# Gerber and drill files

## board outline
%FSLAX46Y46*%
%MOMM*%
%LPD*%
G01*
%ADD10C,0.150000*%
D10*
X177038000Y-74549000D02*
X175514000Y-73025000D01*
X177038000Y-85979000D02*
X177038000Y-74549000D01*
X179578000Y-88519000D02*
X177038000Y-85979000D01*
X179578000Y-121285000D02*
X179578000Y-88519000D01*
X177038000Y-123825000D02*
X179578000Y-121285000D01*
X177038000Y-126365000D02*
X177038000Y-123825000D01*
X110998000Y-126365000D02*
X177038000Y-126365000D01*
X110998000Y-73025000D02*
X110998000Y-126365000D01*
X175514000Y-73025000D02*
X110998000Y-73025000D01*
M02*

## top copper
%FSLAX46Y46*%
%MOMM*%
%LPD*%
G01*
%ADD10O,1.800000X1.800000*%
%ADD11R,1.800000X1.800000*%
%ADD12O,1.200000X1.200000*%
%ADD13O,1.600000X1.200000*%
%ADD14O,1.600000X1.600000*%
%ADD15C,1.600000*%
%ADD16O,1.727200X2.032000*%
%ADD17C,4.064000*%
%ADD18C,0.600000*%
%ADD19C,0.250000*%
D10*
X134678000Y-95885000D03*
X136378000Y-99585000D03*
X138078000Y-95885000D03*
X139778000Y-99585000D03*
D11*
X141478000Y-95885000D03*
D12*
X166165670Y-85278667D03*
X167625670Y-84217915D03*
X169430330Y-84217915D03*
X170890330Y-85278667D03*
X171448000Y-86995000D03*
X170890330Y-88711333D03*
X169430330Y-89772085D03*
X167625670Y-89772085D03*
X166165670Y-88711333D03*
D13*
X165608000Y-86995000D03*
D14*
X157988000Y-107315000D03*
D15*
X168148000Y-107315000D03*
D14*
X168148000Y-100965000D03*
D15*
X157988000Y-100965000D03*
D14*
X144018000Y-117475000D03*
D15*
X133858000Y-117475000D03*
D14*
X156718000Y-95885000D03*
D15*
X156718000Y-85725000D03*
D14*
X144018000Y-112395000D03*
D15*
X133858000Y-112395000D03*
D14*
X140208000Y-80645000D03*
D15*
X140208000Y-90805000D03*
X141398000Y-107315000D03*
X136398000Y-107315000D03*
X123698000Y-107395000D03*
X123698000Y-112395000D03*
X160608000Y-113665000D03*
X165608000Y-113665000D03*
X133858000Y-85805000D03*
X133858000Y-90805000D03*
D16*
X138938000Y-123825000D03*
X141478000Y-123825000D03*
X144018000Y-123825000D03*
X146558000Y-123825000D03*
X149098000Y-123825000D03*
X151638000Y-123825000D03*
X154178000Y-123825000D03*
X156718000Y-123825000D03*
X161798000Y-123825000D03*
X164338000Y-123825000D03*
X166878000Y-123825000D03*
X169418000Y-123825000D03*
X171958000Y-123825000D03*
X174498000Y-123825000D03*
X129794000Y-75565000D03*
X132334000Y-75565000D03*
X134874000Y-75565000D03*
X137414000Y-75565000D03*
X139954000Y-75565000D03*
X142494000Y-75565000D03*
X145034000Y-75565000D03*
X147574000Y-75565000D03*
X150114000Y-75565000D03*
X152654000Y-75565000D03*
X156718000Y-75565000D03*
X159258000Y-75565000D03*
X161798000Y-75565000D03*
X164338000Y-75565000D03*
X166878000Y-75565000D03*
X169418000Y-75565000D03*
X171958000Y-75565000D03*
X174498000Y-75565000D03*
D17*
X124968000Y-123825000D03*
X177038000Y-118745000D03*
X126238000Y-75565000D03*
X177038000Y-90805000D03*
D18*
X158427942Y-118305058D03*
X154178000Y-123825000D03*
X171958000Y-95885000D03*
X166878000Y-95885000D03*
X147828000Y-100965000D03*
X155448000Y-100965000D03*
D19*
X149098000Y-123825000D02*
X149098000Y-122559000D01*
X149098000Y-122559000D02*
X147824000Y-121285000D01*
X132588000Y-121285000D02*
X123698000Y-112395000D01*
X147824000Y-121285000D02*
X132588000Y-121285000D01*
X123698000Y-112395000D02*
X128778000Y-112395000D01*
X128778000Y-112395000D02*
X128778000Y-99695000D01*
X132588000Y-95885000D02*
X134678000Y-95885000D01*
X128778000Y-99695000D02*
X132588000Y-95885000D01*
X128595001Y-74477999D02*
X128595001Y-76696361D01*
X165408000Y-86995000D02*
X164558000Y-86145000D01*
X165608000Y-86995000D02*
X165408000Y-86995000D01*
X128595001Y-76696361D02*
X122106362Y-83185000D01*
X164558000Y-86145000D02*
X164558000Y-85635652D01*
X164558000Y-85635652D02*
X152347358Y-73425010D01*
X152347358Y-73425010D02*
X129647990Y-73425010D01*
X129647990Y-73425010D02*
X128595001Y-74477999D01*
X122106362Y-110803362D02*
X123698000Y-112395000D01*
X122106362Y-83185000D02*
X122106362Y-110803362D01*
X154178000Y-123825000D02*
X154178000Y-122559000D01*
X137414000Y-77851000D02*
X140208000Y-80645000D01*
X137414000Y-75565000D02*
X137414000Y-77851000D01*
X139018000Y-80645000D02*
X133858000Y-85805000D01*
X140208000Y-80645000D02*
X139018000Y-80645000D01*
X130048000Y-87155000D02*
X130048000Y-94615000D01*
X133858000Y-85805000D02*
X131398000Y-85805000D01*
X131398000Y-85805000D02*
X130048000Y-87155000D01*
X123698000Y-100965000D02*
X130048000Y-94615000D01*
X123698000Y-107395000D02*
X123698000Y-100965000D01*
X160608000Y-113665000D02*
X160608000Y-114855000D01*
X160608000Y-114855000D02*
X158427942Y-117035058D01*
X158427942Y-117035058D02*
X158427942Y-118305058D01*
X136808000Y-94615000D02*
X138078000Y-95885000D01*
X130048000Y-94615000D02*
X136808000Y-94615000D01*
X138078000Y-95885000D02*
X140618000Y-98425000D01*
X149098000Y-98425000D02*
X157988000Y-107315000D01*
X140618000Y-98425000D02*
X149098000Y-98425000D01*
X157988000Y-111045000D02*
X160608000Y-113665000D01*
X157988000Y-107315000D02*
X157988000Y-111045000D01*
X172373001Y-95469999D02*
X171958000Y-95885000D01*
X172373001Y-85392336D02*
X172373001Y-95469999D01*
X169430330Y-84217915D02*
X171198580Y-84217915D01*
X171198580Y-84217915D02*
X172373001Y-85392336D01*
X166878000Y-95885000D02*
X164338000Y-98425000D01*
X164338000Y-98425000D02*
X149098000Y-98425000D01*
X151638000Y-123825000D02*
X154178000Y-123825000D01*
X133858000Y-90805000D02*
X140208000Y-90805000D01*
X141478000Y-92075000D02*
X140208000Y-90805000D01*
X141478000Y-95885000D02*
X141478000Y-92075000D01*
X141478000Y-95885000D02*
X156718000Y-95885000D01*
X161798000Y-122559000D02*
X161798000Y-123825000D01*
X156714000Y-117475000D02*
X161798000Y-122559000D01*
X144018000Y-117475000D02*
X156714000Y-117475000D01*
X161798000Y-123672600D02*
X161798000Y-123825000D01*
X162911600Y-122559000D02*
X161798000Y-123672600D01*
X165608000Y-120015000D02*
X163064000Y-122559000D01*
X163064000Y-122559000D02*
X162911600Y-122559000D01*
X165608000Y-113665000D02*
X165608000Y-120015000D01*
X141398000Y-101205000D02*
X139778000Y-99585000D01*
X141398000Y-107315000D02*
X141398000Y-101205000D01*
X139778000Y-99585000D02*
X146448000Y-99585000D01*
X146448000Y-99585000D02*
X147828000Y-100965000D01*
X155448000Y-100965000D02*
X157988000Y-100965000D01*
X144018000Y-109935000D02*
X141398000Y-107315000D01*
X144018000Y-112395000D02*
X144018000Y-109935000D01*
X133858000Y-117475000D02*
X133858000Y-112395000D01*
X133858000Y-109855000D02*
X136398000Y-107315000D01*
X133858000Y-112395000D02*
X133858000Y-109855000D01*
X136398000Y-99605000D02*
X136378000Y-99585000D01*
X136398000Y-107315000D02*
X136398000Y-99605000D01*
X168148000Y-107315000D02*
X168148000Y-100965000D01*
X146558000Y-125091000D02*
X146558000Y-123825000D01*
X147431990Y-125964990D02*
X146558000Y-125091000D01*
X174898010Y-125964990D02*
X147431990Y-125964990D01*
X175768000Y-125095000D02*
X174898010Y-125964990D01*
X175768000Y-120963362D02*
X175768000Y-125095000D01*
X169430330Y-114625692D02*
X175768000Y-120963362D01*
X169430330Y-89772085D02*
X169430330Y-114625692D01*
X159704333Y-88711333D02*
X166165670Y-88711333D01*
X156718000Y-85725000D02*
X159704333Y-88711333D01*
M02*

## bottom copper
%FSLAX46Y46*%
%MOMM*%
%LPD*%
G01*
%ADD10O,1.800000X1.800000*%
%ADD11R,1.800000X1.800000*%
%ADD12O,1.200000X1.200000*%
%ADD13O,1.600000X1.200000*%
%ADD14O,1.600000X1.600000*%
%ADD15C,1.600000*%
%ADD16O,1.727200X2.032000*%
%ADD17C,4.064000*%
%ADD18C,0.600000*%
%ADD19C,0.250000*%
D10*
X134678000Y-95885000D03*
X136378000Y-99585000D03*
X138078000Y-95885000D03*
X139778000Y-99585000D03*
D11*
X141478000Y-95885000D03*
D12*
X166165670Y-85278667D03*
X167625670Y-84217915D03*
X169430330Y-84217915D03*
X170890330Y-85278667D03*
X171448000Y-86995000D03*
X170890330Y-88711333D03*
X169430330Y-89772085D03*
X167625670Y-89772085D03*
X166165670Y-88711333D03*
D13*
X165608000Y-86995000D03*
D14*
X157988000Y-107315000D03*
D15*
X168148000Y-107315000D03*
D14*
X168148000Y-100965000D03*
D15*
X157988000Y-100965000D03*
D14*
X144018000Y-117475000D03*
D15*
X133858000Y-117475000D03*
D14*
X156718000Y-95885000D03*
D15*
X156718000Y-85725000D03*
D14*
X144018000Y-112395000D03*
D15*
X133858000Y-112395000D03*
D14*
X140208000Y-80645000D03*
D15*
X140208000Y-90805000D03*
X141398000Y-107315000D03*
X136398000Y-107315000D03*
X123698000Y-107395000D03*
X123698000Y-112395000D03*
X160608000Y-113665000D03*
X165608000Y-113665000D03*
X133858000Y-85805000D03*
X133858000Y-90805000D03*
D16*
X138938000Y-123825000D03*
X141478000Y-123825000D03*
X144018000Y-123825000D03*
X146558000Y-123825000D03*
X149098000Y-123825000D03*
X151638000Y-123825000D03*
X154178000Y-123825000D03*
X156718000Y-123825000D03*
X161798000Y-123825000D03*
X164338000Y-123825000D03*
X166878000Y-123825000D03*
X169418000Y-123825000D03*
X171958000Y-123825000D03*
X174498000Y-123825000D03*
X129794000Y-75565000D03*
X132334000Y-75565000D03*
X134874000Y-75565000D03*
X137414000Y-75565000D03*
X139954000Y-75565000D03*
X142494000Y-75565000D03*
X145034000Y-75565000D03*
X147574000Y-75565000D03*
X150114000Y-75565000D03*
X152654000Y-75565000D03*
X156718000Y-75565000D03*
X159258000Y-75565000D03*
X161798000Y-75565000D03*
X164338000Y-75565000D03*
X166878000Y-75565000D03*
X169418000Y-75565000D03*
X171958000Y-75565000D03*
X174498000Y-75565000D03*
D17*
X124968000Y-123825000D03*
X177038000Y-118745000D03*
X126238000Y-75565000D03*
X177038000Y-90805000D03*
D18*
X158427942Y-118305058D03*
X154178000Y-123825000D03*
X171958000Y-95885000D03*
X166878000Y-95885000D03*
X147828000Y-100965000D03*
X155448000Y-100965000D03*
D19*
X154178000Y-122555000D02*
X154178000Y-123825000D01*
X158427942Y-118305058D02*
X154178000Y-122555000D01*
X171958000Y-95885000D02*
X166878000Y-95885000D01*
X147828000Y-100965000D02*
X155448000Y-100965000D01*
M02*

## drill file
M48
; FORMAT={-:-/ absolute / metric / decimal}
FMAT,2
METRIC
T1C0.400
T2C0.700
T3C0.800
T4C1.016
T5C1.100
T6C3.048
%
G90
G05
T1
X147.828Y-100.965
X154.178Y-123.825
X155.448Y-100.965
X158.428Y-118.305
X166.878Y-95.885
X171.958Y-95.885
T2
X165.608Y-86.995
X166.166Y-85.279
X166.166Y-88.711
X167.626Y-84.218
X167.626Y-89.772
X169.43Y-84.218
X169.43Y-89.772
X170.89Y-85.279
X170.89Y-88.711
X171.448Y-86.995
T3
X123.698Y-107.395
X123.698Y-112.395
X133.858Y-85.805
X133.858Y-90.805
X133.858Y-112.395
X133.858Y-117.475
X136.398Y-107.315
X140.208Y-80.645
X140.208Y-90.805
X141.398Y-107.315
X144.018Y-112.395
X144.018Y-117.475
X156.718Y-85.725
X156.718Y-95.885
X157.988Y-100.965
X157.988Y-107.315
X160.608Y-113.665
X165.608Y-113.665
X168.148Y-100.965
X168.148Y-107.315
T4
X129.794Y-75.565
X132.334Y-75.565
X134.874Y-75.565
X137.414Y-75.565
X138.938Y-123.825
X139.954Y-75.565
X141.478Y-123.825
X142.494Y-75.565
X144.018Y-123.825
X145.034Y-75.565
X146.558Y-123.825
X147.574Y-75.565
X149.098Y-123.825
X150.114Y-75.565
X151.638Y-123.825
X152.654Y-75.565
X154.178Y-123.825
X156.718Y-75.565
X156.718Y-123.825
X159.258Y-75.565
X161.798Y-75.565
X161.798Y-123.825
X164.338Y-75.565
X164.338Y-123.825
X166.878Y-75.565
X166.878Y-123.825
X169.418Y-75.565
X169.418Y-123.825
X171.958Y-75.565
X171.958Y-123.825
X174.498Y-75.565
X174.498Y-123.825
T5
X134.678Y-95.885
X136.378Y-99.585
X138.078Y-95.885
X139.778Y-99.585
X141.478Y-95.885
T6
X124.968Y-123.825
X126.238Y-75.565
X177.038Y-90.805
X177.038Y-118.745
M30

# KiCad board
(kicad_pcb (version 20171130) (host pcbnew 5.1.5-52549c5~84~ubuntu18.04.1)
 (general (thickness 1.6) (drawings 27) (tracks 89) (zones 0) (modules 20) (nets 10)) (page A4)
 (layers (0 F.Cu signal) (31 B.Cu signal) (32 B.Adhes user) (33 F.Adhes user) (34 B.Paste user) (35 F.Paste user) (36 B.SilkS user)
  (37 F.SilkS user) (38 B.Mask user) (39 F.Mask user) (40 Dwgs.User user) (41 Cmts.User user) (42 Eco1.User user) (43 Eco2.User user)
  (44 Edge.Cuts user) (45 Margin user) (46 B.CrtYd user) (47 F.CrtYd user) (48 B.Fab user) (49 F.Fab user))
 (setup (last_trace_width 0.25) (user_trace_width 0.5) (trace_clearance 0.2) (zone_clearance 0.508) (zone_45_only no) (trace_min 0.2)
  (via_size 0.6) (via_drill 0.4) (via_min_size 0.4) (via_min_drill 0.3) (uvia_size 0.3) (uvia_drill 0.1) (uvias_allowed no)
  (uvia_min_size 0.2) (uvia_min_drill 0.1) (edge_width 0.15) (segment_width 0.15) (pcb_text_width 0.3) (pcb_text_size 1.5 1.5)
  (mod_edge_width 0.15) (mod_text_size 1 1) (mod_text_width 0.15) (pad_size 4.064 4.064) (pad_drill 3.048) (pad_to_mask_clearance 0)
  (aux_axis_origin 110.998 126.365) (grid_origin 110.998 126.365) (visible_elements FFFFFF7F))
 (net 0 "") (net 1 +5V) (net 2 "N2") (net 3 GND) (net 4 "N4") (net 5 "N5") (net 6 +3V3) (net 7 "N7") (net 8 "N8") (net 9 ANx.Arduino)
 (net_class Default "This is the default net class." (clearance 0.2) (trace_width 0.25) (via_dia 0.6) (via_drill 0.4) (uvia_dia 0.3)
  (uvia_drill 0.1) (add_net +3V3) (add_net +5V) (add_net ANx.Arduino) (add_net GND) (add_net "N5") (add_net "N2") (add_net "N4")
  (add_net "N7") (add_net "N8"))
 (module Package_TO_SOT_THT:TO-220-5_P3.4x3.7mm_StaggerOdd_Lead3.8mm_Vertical (layer F.Cu) (at 141.478 95.885 180)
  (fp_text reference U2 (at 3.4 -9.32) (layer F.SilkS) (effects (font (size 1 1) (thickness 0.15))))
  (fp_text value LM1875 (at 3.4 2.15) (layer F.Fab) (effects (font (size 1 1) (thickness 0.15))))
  (pad 5 thru_hole oval (at 6.8 0 180) (size 1.8 1.8) (drill 1.1) (layers *.Cu *.Mask) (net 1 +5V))
  (pad 4 thru_hole oval (at 5.1 -3.7 180) (size 1.8 1.8) (drill 1.1) (layers *.Cu *.Mask) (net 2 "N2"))
  (pad 3 thru_hole oval (at 3.4 0 180) (size 1.8 1.8) (drill 1.1) (layers *.Cu *.Mask) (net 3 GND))
  (pad 2 thru_hole oval (at 1.7 -3.7 180) (size 1.8 1.8) (drill 1.1) (layers *.Cu *.Mask) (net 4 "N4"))
  (pad 1 thru_hole rect (at 0 0 180) (size 1.8 1.8) (drill 1.1) (layers *.Cu *.Mask) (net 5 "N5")))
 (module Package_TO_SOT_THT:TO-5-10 (layer F.Cu) (at 165.608 86.995)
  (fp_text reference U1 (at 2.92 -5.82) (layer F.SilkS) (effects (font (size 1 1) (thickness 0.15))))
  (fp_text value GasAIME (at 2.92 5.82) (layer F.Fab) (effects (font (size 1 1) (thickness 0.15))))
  (pad 10 thru_hole oval (at 0.55767 -1.716333) (size 1.2 1.2) (drill 0.7) (layers *.Cu *.Mask))
  (pad 9 thru_hole oval (at 2.01767 -2.777085) (size 1.2 1.2) (drill 0.7) (layers *.Cu *.Mask))
  (pad 8 thru_hole oval (at 3.82233 -2.777085) (size 1.2 1.2) (drill 0.7) (layers *.Cu *.Mask) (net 3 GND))
  (pad 7 thru_hole oval (at 5.28233 -1.716333) (size 1.2 1.2) (drill 0.7) (layers *.Cu *.Mask))
  (pad 6 thru_hole oval (at 5.84 0) (size 1.2 1.2) (drill 0.7) (layers *.Cu *.Mask))
  (pad 5 thru_hole oval (at 5.28233 1.716333) (size 1.2 1.2) (drill 0.7) (layers *.Cu *.Mask))
  (pad 4 thru_hole oval (at 3.82233 2.777085) (size 1.2 1.2) (drill 0.7) (layers *.Cu *.Mask) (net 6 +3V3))
  (pad 3 thru_hole oval (at 2.01767 2.777085) (size 1.2 1.2) (drill 0.7) (layers *.Cu *.Mask))
  (pad 2 thru_hole oval (at 0.55767 1.716333) (size 1.2 1.2) (drill 0.7) (layers *.Cu *.Mask) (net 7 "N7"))
  (pad 1 thru_hole oval (at 0 0) (size 1.6 1.2) (drill 0.7) (layers *.Cu *.Mask) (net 1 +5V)))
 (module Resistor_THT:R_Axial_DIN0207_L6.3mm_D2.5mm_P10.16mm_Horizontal (layer F.Cu) (at 168.148 107.315 180)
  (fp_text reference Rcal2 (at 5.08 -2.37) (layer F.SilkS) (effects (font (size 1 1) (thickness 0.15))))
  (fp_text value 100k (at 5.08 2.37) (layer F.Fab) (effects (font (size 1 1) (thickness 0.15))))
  (pad 2 thru_hole oval (at 10.16 0 180) (size 1.6 1.6) (drill 0.8) (layers *.Cu *.Mask) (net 3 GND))
  (pad 1 thru_hole circle (at 0 0 180) (size 1.6 1.6) (drill 0.8) (layers *.Cu *.Mask) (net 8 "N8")))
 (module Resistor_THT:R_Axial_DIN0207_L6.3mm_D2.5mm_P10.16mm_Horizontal (layer F.Cu) (at 157.988 100.965)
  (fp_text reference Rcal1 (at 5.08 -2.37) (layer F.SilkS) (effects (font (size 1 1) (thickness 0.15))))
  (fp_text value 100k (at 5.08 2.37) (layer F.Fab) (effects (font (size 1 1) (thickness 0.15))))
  (pad 2 thru_hole oval (at 10.16 0) (size 1.6 1.6) (drill 0.8) (layers *.Cu *.Mask) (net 8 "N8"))
  (pad 1 thru_hole circle (at 0 0) (size 1.6 1.6) (drill 0.8) (layers *.Cu *.Mask) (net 4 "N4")))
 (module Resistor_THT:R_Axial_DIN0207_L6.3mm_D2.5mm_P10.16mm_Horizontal (layer F.Cu) (at 133.858 117.475)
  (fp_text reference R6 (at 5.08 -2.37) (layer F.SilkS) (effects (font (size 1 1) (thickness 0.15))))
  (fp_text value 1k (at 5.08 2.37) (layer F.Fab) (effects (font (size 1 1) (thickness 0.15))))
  (pad 2 thru_hole oval (at 10.16 0) (size 1.6 1.6) (drill 0.8) (layers *.Cu *.Mask) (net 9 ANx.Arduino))
  (pad 1 thru_hole circle (at 0 0) (size 1.6 1.6) (drill 0.8) (layers *.Cu *.Mask) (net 2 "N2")))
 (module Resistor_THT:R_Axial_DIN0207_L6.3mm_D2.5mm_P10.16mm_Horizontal (layer F.Cu) (at 156.718 85.725 270)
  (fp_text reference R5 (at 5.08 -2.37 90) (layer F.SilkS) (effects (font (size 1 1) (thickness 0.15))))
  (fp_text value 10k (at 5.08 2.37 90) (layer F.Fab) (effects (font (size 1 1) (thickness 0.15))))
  (pad 2 thru_hole oval (at 10.16 0 270) (size 1.6 1.6) (drill 0.8) (layers *.Cu *.Mask) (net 5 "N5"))
  (pad 1 thru_hole circle (at 0 0 270) (size 1.6 1.6) (drill 0.8) (layers *.Cu *.Mask) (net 7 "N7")))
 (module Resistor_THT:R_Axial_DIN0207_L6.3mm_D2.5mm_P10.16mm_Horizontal (layer F.Cu) (at 133.858 112.395)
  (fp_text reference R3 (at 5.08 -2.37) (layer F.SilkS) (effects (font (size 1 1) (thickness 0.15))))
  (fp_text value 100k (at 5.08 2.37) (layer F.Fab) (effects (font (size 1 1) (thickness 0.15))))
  (pad 2 thru_hole oval (at 10.16 0) (size 1.6 1.6) (drill 0.8) (layers *.Cu *.Mask) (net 4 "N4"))
  (pad 1 thru_hole circle (at 0 0) (size 1.6 1.6) (drill 0.8) (layers *.Cu *.Mask) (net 2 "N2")))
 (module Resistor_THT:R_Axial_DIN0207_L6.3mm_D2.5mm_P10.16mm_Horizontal (layer F.Cu) (at 140.208 90.805 90)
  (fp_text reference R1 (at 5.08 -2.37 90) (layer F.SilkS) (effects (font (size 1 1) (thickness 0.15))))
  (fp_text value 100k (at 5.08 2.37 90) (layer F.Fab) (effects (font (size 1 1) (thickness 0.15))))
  (pad 2 thru_hole oval (at 10.16 0 90) (size 1.6 1.6) (drill 0.8) (layers *.Cu *.Mask) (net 3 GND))
  (pad 1 thru_hole circle (at 0 0 90) (size 1.6 1.6) (drill 0.8) (layers *.Cu *.Mask) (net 5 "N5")))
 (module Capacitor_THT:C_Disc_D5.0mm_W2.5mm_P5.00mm (layer F.Cu) (at 136.398 107.315)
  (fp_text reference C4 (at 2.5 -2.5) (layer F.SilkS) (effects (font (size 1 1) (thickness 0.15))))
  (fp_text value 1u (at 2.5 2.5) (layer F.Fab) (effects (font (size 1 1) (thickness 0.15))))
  (pad 2 thru_hole circle (at 5 0) (size 1.6 1.6) (drill 0.8) (layers *.Cu *.Mask) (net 4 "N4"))
  (pad 1 thru_hole circle (at 0 0) (size 1.6 1.6) (drill 0.8) (layers *.Cu *.Mask) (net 2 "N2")))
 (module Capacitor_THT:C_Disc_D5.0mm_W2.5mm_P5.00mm (layer F.Cu) (at 123.698 112.395 90)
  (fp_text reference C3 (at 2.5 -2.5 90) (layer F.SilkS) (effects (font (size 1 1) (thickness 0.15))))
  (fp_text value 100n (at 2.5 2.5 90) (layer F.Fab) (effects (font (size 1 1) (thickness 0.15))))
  (pad 2 thru_hole circle (at 5 0 90) (size 1.6 1.6) (drill 0.8) (layers *.Cu *.Mask) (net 3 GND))
  (pad 1 thru_hole circle (at 0 0 90) (size 1.6 1.6) (drill 0.8) (layers *.Cu *.Mask) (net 1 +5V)))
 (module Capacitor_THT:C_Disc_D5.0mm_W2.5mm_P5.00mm (layer F.Cu) (at 165.608 113.665 180)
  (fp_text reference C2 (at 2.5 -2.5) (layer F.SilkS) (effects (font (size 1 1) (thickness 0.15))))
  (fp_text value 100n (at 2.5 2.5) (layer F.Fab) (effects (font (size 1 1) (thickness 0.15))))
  (pad 2 thru_hole circle (at 5 0 180) (size 1.6 1.6) (drill 0.8) (layers *.Cu *.Mask) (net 3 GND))
  (pad 1 thru_hole circle (at 0 0 180) (size 1.6 1.6) (drill 0.8) (layers *.Cu *.Mask) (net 9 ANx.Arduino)))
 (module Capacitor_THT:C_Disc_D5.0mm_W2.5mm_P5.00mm (layer F.Cu) (at 133.858 90.805 90)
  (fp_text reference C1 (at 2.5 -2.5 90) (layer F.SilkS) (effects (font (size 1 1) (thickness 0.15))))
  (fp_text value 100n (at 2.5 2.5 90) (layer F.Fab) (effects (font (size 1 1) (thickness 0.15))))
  (pad 2 thru_hole circle (at 5 0 90) (size 1.6 1.6) (drill 0.8) (layers *.Cu *.Mask) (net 3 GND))
  (pad 1 thru_hole circle (at 0 0 90) (size 1.6 1.6) (drill 0.8) (layers *.Cu *.Mask) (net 5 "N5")))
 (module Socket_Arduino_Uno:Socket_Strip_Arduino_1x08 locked (layer F.Cu) (at 138.938 123.825)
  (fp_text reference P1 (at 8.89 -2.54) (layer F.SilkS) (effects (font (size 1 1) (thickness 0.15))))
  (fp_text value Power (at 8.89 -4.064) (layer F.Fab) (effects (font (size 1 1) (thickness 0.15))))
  (pad 1 thru_hole oval (at 0 0) (size 1.7272 2.032) (drill 1.016) (layers *.Cu *.Mask F.SilkS))
  (pad 2 thru_hole oval (at 2.54 0) (size 1.7272 2.032) (drill 1.016) (layers *.Cu *.Mask F.SilkS))
  (pad 3 thru_hole oval (at 5.08 0) (size 1.7272 2.032) (drill 1.016) (layers *.Cu *.Mask F.SilkS))
  (pad 4 thru_hole oval (at 7.62 0) (size 1.7272 2.032) (drill 1.016) (layers *.Cu *.Mask F.SilkS) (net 6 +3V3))
  (pad 5 thru_hole oval (at 10.16 0) (size 1.7272 2.032) (drill 1.016) (layers *.Cu *.Mask F.SilkS) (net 1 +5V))
  (pad 6 thru_hole oval (at 12.7 0) (size 1.7272 2.032) (drill 1.016) (layers *.Cu *.Mask F.SilkS) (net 3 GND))
  (pad 7 thru_hole oval (at 15.24 0) (size 1.7272 2.032) (drill 1.016) (layers *.Cu *.Mask F.SilkS) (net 3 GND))
  (pad 8 thru_hole oval (at 17.78 0) (size 1.7272 2.032) (drill 1.016) (layers *.Cu *.Mask F.SilkS)))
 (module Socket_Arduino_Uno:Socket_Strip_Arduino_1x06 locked (layer F.Cu) (at 161.798 123.825)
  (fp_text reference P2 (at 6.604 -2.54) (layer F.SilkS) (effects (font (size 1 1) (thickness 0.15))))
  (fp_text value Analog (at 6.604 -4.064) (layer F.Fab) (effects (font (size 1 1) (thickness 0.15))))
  (pad 1 thru_hole oval (at 0 0) (size 1.7272 2.032) (drill 1.016) (layers *.Cu *.Mask F.SilkS) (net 9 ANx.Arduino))
  (pad 2 thru_hole oval (at 2.54 0) (size 1.7272 2.032) (drill 1.016) (layers *.Cu *.Mask F.SilkS))
  (pad 3 thru_hole oval (at 5.08 0) (size 1.7272 2.032) (drill 1.016) (layers *.Cu *.Mask F.SilkS))
  (pad 4 thru_hole oval (at 7.62 0) (size 1.7272 2.032) (drill 1.016) (layers *.Cu *.Mask F.SilkS))
  (pad 5 thru_hole oval (at 10.16 0) (size 1.7272 2.032) (drill 1.016) (layers *.Cu *.Mask F.SilkS))
  (pad 6 thru_hole oval (at 12.7 0) (size 1.7272 2.032) (drill 1.016) (layers *.Cu *.Mask F.SilkS)))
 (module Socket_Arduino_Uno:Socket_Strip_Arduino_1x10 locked (layer F.Cu) (at 129.794 75.565)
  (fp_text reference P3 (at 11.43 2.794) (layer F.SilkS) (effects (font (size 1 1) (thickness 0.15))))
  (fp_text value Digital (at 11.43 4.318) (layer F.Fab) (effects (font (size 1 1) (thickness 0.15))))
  (pad 1 thru_hole oval (at 0 0) (size 1.7272 2.032) (drill 1.016) (layers *.Cu *.Mask F.SilkS))
  (pad 2 thru_hole oval (at 2.54 0) (size 1.7272 2.032) (drill 1.016) (layers *.Cu *.Mask F.SilkS))
  (pad 3 thru_hole oval (at 5.08 0) (size 1.7272 2.032) (drill 1.016) (layers *.Cu *.Mask F.SilkS))
  (pad 4 thru_hole oval (at 7.62 0) (size 1.7272 2.032) (drill 1.016) (layers *.Cu *.Mask F.SilkS) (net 3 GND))
  (pad 5 thru_hole oval (at 10.16 0) (size 1.7272 2.032) (drill 1.016) (layers *.Cu *.Mask F.SilkS))
  (pad 6 thru_hole oval (at 12.7 0) (size 1.7272 2.032) (drill 1.016) (layers *.Cu *.Mask F.SilkS))
  (pad 7 thru_hole oval (at 15.24 0) (size 1.7272 2.032) (drill 1.016) (layers *.Cu *.Mask F.SilkS))
  (pad 8 thru_hole oval (at 17.78 0) (size 1.7272 2.032) (drill 1.016) (layers *.Cu *.Mask F.SilkS))
  (pad 9 thru_hole oval (at 20.32 0) (size 1.7272 2.032) (drill 1.016) (layers *.Cu *.Mask F.SilkS))
  (pad 10 thru_hole oval (at 22.86 0) (size 1.7272 2.032) (drill 1.016) (layers *.Cu *.Mask F.SilkS)))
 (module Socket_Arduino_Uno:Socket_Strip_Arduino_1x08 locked (layer F.Cu) (at 156.718 75.565)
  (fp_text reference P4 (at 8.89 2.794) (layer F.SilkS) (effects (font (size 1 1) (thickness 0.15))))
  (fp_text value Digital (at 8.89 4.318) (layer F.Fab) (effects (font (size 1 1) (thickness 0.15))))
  (pad 1 thru_hole oval (at 0 0) (size 1.7272 2.032) (drill 1.016) (layers *.Cu *.Mask F.SilkS))
  (pad 2 thru_hole oval (at 2.54 0) (size 1.7272 2.032) (drill 1.016) (layers *.Cu *.Mask F.SilkS))
  (pad 3 thru_hole oval (at 5.08 0) (size 1.7272 2.032) (drill 1.016) (layers *.Cu *.Mask F.SilkS))
  (pad 4 thru_hole oval (at 7.62 0) (size 1.7272 2.032) (drill 1.016) (layers *.Cu *.Mask F.SilkS))
  (pad 5 thru_hole oval (at 10.16 0) (size 1.7272 2.032) (drill 1.016) (layers *.Cu *.Mask F.SilkS))
  (pad 6 thru_hole oval (at 12.7 0) (size 1.7272 2.032) (drill 1.016) (layers *.Cu *.Mask F.SilkS))
  (pad 7 thru_hole oval (at 15.24 0) (size 1.7272 2.032) (drill 1.016) (layers *.Cu *.Mask F.SilkS))
  (pad 8 thru_hole oval (at 17.78 0) (size 1.7272 2.032) (drill 1.016) (layers *.Cu *.Mask F.SilkS)))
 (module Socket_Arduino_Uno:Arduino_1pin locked (layer F.Cu) (at 124.968 123.825)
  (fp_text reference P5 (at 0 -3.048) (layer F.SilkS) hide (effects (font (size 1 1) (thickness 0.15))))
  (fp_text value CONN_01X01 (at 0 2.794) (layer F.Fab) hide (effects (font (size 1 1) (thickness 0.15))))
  (pad 1 thru_hole circle (at 0 0) (size 4.064 4.064) (drill 3.048) (layers *.Cu *.Mask F.SilkS)))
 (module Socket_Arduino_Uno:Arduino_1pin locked (layer F.Cu) (at 177.038 118.745)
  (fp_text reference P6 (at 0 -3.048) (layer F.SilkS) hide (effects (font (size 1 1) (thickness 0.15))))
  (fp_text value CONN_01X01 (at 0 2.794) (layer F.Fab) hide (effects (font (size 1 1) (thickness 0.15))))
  (pad 1 thru_hole circle (at 0 0) (size 4.064 4.064) (drill 3.048) (layers *.Cu *.Mask F.SilkS)))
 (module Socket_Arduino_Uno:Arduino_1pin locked (layer F.Cu) (at 126.238 75.565)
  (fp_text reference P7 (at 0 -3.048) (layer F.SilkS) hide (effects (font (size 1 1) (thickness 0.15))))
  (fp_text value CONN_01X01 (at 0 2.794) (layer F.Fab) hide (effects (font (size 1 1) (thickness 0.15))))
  (pad 1 thru_hole circle (at 0 0) (size 4.064 4.064) (drill 3.048) (layers *.Cu *.Mask F.SilkS)))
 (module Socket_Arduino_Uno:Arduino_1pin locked (layer F.Cu) (at 177.038 90.805)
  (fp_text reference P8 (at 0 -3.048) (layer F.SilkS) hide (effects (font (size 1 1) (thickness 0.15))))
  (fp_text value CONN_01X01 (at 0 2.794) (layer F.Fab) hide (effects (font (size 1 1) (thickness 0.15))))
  (pad 1 thru_hole circle (at 0 0) (size 4.064 4.064) (drill 3.048) (layers *.Cu *.Mask F.SilkS)))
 (gr_line (start 177.038 74.549) (end 175.514 73.025) (angle 90) (layer Edge.Cuts) (width 0.15))
 (gr_line (start 177.038 85.979) (end 177.038 74.549) (angle 90) (layer Edge.Cuts) (width 0.15))
 (gr_line (start 179.578 88.519) (end 177.038 85.979) (angle 90) (layer Edge.Cuts) (width 0.15))
 (gr_line (start 179.578 121.285) (end 179.578 88.519) (angle 90) (layer Edge.Cuts) (width 0.15))
 (gr_line (start 177.038 123.825) (end 179.578 121.285) (angle 90) (layer Edge.Cuts) (width 0.15))
 (gr_line (start 177.038 126.365) (end 177.038 123.825) (angle 90) (layer Edge.Cuts) (width 0.15))
 (gr_line (start 110.998 126.365) (end 177.038 126.365) (angle 90) (layer Edge.Cuts) (width 0.15))
 (gr_line (start 110.998 73.025) (end 110.998 126.365) (angle 90) (layer Edge.Cuts) (width 0.15))
 (gr_line (start 175.514 73.025) (end 110.998 73.025) (angle 90) (layer Edge.Cuts) (width 0.15))
 (segment (start 149.098 123.825) (end 149.098 122.559) (width 0.25) (layer F.Cu) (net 1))
 (segment (start 149.098 122.559) (end 147.824 121.285) (width 0.25) (layer F.Cu) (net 1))
 (segment (start 132.588 121.285) (end 123.698 112.395) (width 0.25) (layer F.Cu) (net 1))
 (segment (start 147.824 121.285) (end 132.588 121.285) (width 0.25) (layer F.Cu) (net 1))
 (segment (start 123.698 112.395) (end 128.778 112.395) (width 0.25) (layer F.Cu) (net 1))
 (segment (start 128.778 112.395) (end 128.778 99.695) (width 0.25) (layer F.Cu) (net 1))
 (segment (start 132.588 95.885) (end 134.678 95.885) (width 0.25) (layer F.Cu) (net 1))
 (segment (start 128.778 99.695) (end 132.588 95.885) (width 0.25) (layer F.Cu) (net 1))
 (segment (start 128.595001 74.477999) (end 128.595001 76.696361) (width 0.25) (layer F.Cu) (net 1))
 (segment (start 165.408 86.995) (end 164.558 86.145) (width 0.25) (layer F.Cu) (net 1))
 (segment (start 165.608 86.995) (end 165.408 86.995) (width 0.25) (layer F.Cu) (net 1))
 (segment (start 128.595001 76.696361) (end 122.106362 83.185) (width 0.25) (layer F.Cu) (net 1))
 (segment (start 164.558 86.145) (end 164.558 85.635652) (width 0.25) (layer F.Cu) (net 1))
 (segment (start 164.558 85.635652) (end 152.347358 73.42501) (width 0.25) (layer F.Cu) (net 1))
 (segment (start 152.347358 73.42501) (end 129.64799 73.42501) (width 0.25) (layer F.Cu) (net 1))
 (segment (start 129.64799 73.42501) (end 128.595001 74.477999) (width 0.25) (layer F.Cu) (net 1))
 (segment (start 122.106362 110.803362) (end 123.698 112.395) (width 0.25) (layer F.Cu) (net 1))
 (segment (start 122.106362 83.185) (end 122.106362 110.803362) (width 0.25) (layer F.Cu) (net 1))
 (segment (start 154.178 123.825) (end 154.178 122.559) (width 0.25) (layer F.Cu) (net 3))
 (segment (start 137.414 77.851) (end 140.208 80.645) (width 0.25) (layer F.Cu) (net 3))
 (segment (start 137.414 75.565) (end 137.414 77.851) (width 0.25) (layer F.Cu) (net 3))
 (segment (start 139.018 80.645) (end 133.858 85.805) (width 0.25) (layer F.Cu) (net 3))
 (segment (start 140.208 80.645) (end 139.018 80.645) (width 0.25) (layer F.Cu) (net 3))
 (segment (start 130.048 87.155) (end 130.048 94.615) (width 0.25) (layer F.Cu) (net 3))
 (segment (start 133.858 85.805) (end 131.398 85.805) (width 0.25) (layer F.Cu) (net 3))
 (segment (start 131.398 85.805) (end 130.048 87.155) (width 0.25) (layer F.Cu) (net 3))
 (segment (start 123.698 100.965) (end 130.048 94.615) (width 0.25) (layer F.Cu) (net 3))
 (segment (start 123.698 107.395) (end 123.698 100.965) (width 0.25) (layer F.Cu) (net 3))
 (segment (start 160.608 113.665) (end 160.608 114.855) (width 0.25) (layer F.Cu) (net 3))
 (via (at 158.427942 118.305058) (size 0.6) (drill 0.4) (layers F.Cu B.Cu) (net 3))
 (segment (start 160.608 114.855) (end 158.427942 117.035058) (width 0.25) (layer F.Cu) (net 3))
 (segment (start 158.427942 117.035058) (end 158.427942 118.305058) (width 0.25) (layer F.Cu) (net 3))
 (segment (start 154.178 122.555) (end 154.178 123.825) (width 0.25) (layer B.Cu) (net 3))
 (segment (start 158.427942 118.305058) (end 154.178 122.555) (width 0.25) (layer B.Cu) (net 3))
 (via (at 154.178 123.825) (size 0.6) (drill 0.4) (layers F.Cu B.Cu) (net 3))
 (segment (start 136.808 94.615) (end 138.078 95.885) (width 0.25) (layer F.Cu) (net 3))
 (segment (start 130.048 94.615) (end 136.808 94.615) (width 0.25) (layer F.Cu) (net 3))
 (segment (start 138.078 95.885) (end 140.618 98.425) (width 0.25) (layer F.Cu) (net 3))
 (segment (start 149.098 98.425) (end 157.988 107.315) (width 0.25) (layer F.Cu) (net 3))
 (segment (start 140.618 98.425) (end 149.098 98.425) (width 0.25) (layer F.Cu) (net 3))
 (segment (start 157.988 111.045) (end 160.608 113.665) (width 0.25) (layer F.Cu) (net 3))
 (segment (start 157.988 107.315) (end 157.988 111.045) (width 0.25) (layer F.Cu) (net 3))
 (via (at 171.958 95.885) (size 0.6) (drill 0.4) (layers F.Cu B.Cu) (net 3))
 (segment (start 172.373001 95.469999) (end 171.958 95.885) (width 0.25) (layer F.Cu) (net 3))
 (segment (start 172.373001 85.392336) (end 172.373001 95.469999) (width 0.25) (layer F.Cu) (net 3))
 (segment (start 169.43033 84.217915) (end 171.19858 84.217915) (width 0.25) (layer F.Cu) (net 3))
 (segment (start 171.19858 84.217915) (end 172.373001 85.392336) (width 0.25) (layer F.Cu) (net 3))
 (segment (start 171.958 95.885) (end 166.878 95.885) (width 0.25) (layer B.Cu) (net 3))
 (via (at 166.878 95.885) (size 0.6) (drill 0.4) (layers F.Cu B.Cu) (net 3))
 (segment (start 166.878 95.885) (end 164.338 98.425) (width 0.25) (layer F.Cu) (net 3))
 (segment (start 164.338 98.425) (end 149.098 98.425) (width 0.25) (layer F.Cu) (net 3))
 (segment (start 151.638 123.825) (end 154.178 123.825) (width 0.25) (layer F.Cu) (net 3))
 (segment (start 133.858 90.805) (end 140.208 90.805) (width 0.25) (layer F.Cu) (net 5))
 (segment (start 141.478 92.075) (end 140.208 90.805) (width 0.25) (layer F.Cu) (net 5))
 (segment (start 141.478 95.885) (end 141.478 92.075) (width 0.25) (layer F.Cu) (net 5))
 (segment (start 141.478 95.885) (end 156.718 95.885) (width 0.25) (layer F.Cu) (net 5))
 (segment (start 161.798 122.559) (end 161.798 123.825) (width 0.25) (layer F.Cu) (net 9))
 (segment (start 156.714 117.475) (end 161.798 122.559) (width 0.25) (layer F.Cu) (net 9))
 (segment (start 144.018 117.475) (end 156.714 117.475) (width 0.25) (layer F.Cu) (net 9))
 (segment (start 161.798 123.6726) (end 161.798 123.825) (width 0.25) (layer F.Cu) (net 9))
 (segment (start 162.9116 122.559) (end 161.798 123.6726) (width 0.25) (layer F.Cu) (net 9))
 (segment (start 165.608 120.015) (end 163.064 122.559) (width 0.25) (layer F.Cu) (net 9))
 (segment (start 163.064 122.559) (end 162.9116 122.559) (width 0.25) (layer F.Cu) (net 9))
 (segment (start 165.608 113.665) (end 165.608 120.015) (width 0.25) (layer F.Cu) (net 9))
 (segment (start 141.398 101.205) (end 139.778 99.585) (width 0.25) (layer F.Cu) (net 4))
 (segment (start 141.398 107.315) (end 141.398 101.205) (width 0.25) (layer F.Cu) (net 4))
 (segment (start 139.778 99.585) (end 146.448 99.585) (width 0.25) (layer F.Cu) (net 4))
 (segment (start 146.448 99.585) (end 147.828 100.965) (width 0.25) (layer F.Cu) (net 4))
 (via (at 147.828 100.965) (size 0.6) (drill 0.4) (layers F.Cu B.Cu) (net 4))
 (segment (start 147.828 100.965) (end 155.448 100.965) (width 0.25) (layer B.Cu) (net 4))
 (via (at 155.448 100.965) (size 0.6) (drill 0.4) (layers F.Cu B.Cu) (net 4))
 (segment (start 155.448 100.965) (end 157.988 100.965) (width 0.25) (layer F.Cu) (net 4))
 (segment (start 144.018 109.935) (end 141.398 107.315) (width 0.25) (layer F.Cu) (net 4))
 (segment (start 144.018 112.395) (end 144.018 109.935) (width 0.25) (layer F.Cu) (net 4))
 (segment (start 133.858 117.475) (end 133.858 112.395) (width 0.25) (layer F.Cu) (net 2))
 (segment (start 133.858 109.855) (end 136.398 107.315) (width 0.25) (layer F.Cu) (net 2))
 (segment (start 133.858 112.395) (end 133.858 109.855) (width 0.25) (layer F.Cu) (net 2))
 (segment (start 136.398 99.605) (end 136.378 99.585) (width 0.25) (layer F.Cu) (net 2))
 (segment (start 136.398 107.315) (end 136.398 99.605) (width 0.25) (layer F.Cu) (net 2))
 (segment (start 168.148 107.315) (end 168.148 100.965) (width 0.25) (layer F.Cu) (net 8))
 (segment (start 146.558 125.091) (end 146.558 123.825) (width 0.25) (layer F.Cu) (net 6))
 (segment (start 147.43199 125.96499) (end 146.558 125.091) (width 0.25) (layer F.Cu) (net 6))
 (segment (start 174.89801 125.96499) (end 147.43199 125.96499) (width 0.25) (layer F.Cu) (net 6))
 (segment (start 175.768 125.095) (end 174.89801 125.96499) (width 0.25) (layer F.Cu) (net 6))
 (segment (start 175.768 120.963362) (end 175.768 125.095) (width 0.25) (layer F.Cu) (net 6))
 (segment (start 169.43033 114.625692) (end 175.768 120.963362) (width 0.25) (layer F.Cu) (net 6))
 (segment (start 169.43033 89.772085) (end 169.43033 114.625692) (width 0.25) (layer F.Cu) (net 6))
 (segment (start 159.704333 88.711333) (end 166.16567 88.711333) (width 0.25) (layer F.Cu) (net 7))
 (segment (start 156.718 85.725) (end 159.704333 88.711333) (width 0.25) (layer F.Cu) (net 7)))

